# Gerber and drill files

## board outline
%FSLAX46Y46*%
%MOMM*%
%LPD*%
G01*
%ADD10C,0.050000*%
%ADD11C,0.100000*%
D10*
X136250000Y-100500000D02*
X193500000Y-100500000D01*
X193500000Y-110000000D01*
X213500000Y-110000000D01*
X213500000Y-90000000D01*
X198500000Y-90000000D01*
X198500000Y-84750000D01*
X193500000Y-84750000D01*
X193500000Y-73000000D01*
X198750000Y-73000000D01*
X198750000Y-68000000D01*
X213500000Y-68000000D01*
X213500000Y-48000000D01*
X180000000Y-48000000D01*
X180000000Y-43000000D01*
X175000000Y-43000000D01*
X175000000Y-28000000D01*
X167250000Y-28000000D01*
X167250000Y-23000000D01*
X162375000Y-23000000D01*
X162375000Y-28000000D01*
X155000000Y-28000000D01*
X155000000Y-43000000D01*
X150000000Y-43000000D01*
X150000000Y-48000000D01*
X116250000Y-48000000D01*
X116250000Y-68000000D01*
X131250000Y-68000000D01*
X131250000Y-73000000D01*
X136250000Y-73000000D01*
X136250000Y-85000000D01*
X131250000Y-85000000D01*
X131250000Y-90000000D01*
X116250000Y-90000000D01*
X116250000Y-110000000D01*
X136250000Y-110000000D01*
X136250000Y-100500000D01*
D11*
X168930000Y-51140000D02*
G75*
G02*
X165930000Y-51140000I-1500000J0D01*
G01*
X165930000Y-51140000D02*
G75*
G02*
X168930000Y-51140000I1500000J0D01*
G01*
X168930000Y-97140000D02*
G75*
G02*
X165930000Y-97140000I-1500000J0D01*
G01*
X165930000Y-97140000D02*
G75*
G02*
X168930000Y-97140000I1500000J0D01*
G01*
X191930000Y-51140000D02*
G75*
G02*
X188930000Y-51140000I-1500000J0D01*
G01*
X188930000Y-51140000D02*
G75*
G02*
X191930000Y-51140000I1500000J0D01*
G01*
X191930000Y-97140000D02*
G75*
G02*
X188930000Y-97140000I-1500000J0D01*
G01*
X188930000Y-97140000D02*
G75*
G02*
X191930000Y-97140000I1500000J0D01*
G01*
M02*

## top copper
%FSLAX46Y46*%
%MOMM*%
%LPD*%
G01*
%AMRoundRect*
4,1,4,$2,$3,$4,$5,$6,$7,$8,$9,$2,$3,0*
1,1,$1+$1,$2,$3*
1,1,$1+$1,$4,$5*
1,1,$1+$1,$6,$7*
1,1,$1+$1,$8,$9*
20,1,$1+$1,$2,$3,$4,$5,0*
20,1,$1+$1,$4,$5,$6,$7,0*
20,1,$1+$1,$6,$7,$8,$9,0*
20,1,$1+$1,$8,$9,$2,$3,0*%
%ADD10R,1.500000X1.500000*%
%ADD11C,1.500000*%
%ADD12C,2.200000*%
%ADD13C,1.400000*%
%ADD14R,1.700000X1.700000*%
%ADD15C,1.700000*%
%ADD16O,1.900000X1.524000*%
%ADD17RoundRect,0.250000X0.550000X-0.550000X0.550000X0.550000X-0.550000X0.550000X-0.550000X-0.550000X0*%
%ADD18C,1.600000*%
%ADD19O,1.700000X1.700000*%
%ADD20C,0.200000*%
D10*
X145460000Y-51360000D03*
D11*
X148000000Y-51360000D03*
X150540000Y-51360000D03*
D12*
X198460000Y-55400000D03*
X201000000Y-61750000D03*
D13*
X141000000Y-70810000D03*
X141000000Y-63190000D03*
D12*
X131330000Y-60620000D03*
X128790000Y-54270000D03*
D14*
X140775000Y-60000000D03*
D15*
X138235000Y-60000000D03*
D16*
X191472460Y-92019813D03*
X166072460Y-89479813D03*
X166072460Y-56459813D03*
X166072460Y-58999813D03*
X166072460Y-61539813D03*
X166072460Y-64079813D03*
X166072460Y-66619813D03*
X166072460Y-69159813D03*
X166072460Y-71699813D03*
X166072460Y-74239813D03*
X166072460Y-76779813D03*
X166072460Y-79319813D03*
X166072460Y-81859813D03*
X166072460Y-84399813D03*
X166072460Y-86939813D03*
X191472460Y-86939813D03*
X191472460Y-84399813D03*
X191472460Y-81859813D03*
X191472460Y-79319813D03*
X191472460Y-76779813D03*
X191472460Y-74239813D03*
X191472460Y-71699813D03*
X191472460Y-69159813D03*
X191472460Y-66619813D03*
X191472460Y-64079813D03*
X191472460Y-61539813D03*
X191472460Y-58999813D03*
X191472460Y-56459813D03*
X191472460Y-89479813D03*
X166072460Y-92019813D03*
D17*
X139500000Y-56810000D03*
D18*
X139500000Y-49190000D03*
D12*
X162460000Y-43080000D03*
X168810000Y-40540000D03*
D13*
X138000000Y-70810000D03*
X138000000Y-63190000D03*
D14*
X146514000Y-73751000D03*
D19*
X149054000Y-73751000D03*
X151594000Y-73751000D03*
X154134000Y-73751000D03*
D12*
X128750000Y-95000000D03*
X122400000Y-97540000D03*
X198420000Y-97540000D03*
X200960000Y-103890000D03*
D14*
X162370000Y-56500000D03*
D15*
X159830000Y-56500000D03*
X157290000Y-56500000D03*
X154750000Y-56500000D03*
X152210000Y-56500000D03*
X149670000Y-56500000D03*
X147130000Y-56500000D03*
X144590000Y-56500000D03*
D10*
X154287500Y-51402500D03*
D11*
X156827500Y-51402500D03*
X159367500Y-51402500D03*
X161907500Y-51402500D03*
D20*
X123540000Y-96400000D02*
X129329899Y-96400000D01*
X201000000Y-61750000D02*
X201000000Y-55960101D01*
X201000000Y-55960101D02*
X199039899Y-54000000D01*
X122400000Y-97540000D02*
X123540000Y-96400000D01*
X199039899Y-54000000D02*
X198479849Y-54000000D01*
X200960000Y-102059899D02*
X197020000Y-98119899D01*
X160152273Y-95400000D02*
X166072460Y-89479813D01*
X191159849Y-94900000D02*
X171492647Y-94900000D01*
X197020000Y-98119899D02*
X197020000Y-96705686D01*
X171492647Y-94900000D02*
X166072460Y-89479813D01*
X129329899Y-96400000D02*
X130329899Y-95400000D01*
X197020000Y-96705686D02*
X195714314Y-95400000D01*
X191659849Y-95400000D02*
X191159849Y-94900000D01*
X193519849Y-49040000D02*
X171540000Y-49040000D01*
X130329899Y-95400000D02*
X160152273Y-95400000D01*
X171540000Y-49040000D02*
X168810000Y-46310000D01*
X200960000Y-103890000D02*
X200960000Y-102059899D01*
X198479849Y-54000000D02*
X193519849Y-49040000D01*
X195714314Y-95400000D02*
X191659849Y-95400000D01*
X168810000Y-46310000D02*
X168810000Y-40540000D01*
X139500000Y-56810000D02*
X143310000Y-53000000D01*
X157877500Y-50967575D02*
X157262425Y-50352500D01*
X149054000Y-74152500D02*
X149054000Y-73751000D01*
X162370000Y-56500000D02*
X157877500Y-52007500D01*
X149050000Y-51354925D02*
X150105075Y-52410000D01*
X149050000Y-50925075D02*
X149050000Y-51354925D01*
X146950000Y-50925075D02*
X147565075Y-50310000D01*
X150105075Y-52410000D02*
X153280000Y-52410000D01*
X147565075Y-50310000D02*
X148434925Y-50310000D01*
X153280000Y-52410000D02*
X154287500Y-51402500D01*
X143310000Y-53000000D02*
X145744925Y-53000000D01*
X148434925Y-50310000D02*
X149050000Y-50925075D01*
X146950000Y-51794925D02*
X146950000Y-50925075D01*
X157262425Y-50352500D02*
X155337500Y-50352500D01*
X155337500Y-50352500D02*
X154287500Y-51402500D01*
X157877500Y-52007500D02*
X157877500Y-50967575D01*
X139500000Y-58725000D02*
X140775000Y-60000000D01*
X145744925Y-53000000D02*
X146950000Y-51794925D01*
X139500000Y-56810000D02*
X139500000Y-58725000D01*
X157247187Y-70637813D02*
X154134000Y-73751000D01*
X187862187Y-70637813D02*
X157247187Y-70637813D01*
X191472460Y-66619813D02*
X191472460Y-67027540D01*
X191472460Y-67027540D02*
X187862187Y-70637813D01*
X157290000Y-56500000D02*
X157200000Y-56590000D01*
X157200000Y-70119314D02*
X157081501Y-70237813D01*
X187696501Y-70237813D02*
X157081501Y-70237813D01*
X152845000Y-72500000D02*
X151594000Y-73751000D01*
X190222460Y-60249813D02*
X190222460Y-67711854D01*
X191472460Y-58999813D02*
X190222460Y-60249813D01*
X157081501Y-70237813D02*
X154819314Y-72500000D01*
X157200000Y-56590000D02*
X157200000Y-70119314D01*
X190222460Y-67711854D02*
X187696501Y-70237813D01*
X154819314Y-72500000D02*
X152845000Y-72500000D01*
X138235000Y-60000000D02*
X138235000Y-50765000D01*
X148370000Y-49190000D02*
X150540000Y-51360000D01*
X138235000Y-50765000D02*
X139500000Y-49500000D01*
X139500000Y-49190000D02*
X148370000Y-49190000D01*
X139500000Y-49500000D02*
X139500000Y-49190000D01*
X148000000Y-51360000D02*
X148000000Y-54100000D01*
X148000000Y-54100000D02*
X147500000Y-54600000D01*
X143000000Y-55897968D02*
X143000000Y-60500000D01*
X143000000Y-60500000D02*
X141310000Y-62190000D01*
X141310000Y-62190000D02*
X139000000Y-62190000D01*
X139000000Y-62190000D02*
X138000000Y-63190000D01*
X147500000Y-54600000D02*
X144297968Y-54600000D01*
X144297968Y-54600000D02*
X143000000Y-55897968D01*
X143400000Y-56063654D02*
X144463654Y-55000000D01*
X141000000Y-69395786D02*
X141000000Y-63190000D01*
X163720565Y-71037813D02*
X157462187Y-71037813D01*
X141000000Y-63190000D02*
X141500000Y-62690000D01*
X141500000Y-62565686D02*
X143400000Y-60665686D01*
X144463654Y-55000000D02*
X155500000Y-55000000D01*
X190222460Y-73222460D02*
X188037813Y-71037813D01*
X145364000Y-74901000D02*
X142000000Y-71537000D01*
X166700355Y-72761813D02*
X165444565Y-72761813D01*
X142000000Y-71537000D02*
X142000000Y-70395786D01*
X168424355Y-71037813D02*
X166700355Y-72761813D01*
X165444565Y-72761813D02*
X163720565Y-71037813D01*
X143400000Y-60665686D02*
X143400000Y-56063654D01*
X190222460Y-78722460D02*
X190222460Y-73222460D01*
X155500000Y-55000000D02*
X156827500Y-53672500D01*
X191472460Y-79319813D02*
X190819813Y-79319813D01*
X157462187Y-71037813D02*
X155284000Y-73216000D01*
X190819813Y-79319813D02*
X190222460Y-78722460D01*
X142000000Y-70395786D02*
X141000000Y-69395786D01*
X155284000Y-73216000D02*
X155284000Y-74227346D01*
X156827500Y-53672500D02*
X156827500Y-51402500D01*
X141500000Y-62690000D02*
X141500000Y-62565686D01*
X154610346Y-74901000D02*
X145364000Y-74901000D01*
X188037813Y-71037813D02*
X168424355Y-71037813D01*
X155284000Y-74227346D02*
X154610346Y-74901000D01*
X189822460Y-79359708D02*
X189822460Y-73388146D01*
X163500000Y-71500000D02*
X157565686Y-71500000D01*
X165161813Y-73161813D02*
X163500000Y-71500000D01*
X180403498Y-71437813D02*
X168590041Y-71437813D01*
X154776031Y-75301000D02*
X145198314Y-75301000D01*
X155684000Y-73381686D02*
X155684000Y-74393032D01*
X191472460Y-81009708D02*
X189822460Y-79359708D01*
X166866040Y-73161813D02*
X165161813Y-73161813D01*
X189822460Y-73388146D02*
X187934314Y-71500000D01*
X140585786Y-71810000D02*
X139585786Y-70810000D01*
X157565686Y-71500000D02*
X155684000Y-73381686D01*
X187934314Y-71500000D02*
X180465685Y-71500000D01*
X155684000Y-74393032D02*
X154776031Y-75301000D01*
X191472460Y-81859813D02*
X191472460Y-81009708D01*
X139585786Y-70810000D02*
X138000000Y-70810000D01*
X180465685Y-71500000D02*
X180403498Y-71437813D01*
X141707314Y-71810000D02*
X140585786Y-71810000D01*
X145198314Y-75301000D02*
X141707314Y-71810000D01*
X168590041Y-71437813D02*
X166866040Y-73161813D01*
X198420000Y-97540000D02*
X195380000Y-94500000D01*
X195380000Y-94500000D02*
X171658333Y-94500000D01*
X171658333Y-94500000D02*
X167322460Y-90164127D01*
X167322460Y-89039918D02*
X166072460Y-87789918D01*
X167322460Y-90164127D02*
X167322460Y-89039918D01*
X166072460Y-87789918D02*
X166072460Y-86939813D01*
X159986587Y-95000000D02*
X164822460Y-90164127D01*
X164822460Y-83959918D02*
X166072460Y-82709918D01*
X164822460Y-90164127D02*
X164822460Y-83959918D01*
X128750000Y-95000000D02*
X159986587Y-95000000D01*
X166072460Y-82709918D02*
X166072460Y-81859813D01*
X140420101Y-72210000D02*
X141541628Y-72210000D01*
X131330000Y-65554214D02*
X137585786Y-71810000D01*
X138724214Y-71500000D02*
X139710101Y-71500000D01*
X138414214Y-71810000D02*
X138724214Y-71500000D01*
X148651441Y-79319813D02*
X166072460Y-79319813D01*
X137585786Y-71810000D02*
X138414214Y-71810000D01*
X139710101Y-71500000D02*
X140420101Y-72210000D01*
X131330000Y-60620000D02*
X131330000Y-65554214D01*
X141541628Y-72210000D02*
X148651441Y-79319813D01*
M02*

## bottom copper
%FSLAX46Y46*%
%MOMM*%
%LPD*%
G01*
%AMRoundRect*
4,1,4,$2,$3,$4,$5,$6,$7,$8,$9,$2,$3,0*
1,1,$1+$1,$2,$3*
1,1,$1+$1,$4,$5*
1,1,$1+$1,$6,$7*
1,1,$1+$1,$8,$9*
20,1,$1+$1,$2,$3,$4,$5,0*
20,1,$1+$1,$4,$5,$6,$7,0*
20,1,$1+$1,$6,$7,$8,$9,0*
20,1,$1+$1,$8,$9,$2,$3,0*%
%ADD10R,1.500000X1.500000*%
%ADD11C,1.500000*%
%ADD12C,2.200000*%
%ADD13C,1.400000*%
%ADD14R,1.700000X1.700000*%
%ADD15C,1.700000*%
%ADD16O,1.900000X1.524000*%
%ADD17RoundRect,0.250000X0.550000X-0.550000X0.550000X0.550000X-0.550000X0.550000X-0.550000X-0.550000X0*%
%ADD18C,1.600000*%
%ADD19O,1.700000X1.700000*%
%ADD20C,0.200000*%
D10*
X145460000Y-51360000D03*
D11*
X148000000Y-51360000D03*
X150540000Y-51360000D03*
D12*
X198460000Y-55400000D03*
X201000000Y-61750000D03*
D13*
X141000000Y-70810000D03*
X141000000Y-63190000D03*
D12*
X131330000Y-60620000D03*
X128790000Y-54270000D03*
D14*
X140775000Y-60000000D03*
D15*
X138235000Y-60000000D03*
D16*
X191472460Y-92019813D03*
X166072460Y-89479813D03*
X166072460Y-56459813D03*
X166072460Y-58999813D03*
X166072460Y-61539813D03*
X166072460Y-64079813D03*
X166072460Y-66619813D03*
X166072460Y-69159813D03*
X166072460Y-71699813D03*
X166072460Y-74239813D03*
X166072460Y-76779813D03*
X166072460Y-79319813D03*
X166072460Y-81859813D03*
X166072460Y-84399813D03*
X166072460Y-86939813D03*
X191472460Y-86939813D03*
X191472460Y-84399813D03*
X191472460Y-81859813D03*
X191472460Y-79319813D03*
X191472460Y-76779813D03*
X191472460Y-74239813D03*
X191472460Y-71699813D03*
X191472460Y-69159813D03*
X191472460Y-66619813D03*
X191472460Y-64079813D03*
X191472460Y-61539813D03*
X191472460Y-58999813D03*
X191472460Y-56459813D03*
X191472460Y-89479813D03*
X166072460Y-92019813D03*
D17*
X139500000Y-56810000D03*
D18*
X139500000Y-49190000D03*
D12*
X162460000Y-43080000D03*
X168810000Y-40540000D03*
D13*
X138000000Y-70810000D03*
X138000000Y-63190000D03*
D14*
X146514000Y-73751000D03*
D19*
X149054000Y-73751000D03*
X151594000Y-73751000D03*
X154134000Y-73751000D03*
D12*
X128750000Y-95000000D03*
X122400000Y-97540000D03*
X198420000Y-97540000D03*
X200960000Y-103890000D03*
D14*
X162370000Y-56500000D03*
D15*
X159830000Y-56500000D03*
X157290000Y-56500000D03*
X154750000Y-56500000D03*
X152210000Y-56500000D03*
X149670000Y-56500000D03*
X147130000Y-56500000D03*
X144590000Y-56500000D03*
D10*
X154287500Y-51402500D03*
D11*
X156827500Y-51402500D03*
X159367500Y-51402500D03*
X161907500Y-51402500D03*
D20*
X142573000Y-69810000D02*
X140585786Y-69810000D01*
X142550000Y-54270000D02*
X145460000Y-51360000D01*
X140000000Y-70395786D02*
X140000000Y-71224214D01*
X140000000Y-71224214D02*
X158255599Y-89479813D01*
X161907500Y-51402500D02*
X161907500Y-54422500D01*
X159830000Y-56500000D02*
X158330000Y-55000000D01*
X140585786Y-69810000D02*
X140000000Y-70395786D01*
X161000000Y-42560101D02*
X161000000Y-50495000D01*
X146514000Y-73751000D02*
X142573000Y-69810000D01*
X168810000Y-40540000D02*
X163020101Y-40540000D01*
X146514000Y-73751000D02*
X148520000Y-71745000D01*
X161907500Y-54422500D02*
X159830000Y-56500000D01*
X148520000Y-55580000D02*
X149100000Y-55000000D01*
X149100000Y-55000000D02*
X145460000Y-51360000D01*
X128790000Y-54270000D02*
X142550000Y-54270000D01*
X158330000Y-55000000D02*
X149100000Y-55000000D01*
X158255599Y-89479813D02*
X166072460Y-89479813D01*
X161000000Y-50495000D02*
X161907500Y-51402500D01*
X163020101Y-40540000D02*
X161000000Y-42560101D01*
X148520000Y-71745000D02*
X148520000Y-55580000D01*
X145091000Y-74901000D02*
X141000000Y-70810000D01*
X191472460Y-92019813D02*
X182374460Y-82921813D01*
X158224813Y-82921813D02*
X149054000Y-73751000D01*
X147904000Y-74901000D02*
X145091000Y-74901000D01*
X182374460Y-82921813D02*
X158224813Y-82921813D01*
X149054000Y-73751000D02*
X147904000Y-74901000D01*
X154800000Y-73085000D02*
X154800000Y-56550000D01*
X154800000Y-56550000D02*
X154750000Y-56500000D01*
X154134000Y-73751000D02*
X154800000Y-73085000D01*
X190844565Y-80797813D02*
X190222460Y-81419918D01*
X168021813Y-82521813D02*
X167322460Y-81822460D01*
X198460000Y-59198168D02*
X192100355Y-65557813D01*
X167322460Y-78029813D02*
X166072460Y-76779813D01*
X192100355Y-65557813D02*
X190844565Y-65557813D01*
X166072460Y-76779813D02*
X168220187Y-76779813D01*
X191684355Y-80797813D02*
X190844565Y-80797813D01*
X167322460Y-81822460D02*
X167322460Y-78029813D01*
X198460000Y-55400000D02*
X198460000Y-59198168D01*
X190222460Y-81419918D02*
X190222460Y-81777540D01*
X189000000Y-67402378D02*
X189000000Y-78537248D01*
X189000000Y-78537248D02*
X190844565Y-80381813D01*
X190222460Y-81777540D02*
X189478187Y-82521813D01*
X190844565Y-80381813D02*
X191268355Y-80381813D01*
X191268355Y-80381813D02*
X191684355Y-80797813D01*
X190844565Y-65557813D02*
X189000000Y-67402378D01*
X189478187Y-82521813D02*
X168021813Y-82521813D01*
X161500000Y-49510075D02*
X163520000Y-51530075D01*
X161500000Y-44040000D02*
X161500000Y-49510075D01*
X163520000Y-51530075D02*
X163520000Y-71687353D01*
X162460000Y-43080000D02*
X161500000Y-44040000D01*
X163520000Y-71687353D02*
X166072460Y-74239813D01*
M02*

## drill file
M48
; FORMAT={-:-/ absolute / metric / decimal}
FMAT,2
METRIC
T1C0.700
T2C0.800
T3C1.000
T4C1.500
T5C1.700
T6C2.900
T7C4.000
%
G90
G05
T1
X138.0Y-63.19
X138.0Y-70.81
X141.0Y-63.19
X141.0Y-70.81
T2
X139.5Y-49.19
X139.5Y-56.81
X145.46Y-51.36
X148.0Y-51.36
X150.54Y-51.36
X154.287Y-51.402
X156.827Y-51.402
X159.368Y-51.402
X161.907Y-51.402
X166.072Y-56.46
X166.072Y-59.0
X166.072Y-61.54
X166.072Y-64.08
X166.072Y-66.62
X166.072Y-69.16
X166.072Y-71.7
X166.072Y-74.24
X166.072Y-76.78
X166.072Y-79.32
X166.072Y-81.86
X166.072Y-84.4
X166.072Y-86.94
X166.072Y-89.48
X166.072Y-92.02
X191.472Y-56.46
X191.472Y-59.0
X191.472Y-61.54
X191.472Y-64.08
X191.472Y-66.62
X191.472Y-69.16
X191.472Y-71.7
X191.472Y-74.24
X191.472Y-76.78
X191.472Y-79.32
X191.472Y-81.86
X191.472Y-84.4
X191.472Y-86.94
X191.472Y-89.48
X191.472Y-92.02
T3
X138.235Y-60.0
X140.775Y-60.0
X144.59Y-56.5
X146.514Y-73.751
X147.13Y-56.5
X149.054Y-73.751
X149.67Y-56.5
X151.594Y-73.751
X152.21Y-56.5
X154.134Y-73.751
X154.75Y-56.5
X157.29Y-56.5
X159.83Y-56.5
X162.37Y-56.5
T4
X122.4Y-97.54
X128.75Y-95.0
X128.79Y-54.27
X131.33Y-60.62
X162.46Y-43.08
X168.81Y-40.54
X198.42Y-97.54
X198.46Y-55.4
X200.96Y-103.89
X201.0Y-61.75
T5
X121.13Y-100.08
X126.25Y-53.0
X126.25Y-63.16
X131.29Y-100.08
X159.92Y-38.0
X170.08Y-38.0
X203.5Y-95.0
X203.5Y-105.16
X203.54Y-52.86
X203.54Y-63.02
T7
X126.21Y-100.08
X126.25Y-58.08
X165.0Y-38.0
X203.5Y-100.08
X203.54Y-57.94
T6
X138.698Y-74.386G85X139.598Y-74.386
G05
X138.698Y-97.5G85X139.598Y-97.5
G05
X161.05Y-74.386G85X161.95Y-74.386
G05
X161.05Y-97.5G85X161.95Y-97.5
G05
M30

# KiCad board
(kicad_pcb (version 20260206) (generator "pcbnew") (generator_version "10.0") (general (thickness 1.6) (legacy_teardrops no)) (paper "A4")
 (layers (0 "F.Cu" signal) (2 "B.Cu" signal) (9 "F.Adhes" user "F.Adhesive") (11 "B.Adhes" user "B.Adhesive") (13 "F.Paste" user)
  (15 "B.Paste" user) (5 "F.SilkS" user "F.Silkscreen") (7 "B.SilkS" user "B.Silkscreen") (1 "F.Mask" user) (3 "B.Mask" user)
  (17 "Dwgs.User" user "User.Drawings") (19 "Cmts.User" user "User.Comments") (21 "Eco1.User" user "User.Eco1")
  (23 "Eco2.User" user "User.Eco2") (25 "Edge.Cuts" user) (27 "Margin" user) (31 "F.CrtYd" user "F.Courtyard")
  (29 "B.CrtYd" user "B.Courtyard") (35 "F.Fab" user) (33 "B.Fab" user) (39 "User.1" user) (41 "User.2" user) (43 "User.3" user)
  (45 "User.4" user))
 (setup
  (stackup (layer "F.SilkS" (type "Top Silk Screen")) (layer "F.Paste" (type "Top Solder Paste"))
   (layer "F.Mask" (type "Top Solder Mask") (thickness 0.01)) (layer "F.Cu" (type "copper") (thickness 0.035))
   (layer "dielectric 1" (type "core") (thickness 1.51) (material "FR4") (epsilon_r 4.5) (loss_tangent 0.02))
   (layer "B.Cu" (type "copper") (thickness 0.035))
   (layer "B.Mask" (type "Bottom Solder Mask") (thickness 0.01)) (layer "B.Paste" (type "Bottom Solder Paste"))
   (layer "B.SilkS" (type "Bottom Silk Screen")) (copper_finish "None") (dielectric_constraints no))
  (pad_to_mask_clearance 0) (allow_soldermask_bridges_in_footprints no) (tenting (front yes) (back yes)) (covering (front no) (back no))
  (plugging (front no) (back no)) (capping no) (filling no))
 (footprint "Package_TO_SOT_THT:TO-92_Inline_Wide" (layer "F.Cu") (at 145.46 51.36)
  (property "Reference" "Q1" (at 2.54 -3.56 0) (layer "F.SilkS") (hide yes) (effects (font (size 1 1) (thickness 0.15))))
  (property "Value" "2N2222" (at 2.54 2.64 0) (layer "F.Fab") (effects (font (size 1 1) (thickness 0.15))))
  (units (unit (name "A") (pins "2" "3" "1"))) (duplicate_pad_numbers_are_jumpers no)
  (pad "1" thru_hole rect (at 0 0) (size 1.5 1.5) (drill 0.8) (layers "*.Cu" "*.Mask") (remove_unused_layers no) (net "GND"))
  (pad "2" thru_hole circle (at 2.54 0) (size 1.5 1.5) (drill 0.8) (layers "*.Cu" "*.Mask") (remove_unused_layers no) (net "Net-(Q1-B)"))
  (pad "3" thru_hole circle (at 5.08 0) (size 1.5 1.5) (drill 0.8) (layers "*.Cu" "*.Mask") (remove_unused_layers no) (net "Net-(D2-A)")))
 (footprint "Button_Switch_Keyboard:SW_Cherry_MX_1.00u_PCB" (layer "F.Cu") (at 198.46 55.4 90)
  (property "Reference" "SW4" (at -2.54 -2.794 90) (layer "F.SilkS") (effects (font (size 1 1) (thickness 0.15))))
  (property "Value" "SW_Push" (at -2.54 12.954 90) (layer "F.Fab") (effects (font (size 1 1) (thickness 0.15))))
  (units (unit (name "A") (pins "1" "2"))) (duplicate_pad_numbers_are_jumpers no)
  (pad "" np_thru_hole circle (at -7.62 5.08 90) (size 1.7 1.7) (drill 1.7) (layers "*.Cu" "*.Mask"))
  (pad "" np_thru_hole circle (at -2.54 5.08 90) (size 4 4) (drill 4) (layers "*.Cu" "*.Mask"))
  (pad "" np_thru_hole circle (at 2.54 5.08 90) (size 1.7 1.7) (drill 1.7) (layers "*.Cu" "*.Mask"))
  (pad "1" thru_hole circle (at 0 0 90) (size 2.2 2.2) (drill 1.5) (layers "*.Cu" "*.Mask") (remove_unused_layers no) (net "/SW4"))
  (pad "2" thru_hole circle (at -6.35 2.54 90) (size 2.2 2.2) (drill 1.5) (layers "*.Cu" "*.Mask") (remove_unused_layers no) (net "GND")))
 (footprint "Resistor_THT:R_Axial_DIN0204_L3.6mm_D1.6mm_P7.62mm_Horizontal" (layer "F.Cu") (at 141 70.81 90)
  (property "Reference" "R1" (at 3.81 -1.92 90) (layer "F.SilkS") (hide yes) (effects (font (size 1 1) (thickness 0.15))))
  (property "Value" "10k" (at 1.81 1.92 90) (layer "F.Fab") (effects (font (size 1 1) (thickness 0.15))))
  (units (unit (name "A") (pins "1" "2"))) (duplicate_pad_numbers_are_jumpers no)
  (pad "1" thru_hole circle (at 0 0 90) (size 1.4 1.4) (drill 0.7) (layers "*.Cu" "*.Mask") (remove_unused_layers no) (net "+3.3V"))
  (pad "2" thru_hole circle (at 7.62 0 90) (size 1.4 1.4) (drill 0.7) (layers "*.Cu" "*.Mask") (remove_unused_layers no) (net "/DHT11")))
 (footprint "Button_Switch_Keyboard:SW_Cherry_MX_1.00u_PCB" (layer "F.Cu") (at 131.33 60.62 -90)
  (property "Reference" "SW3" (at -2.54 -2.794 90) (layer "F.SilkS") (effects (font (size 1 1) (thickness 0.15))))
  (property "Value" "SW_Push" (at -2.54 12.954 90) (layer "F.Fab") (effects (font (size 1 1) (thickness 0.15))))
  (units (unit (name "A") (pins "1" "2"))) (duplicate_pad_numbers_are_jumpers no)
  (pad "" np_thru_hole circle (at -7.62 5.08 270) (size 1.7 1.7) (drill 1.7) (layers "*.Cu" "*.Mask"))
  (pad "" np_thru_hole circle (at -2.54 5.08 270) (size 4 4) (drill 4) (layers "*.Cu" "*.Mask"))
  (pad "" np_thru_hole circle (at 2.54 5.08 270) (size 1.7 1.7) (drill 1.7) (layers "*.Cu" "*.Mask"))
  (pad "1" thru_hole circle (at 0 0 270) (size 2.2 2.2) (drill 1.5) (layers "*.Cu" "*.Mask") (remove_unused_layers no) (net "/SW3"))
  (pad "2" thru_hole circle (at -6.35 2.54 270) (size 2.2 2.2) (drill 1.5) (layers "*.Cu" "*.Mask") (remove_unused_layers no) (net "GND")))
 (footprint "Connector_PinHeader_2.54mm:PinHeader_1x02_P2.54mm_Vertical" (layer "F.Cu") (at 140.775 60 -90)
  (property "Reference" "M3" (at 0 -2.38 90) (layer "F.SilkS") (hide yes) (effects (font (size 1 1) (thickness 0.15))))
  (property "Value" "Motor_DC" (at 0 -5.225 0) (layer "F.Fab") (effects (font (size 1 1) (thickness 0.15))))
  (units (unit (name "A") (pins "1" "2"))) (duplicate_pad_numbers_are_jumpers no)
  (pad "1" thru_hole rect (at 0 0 270) (size 1.7 1.7) (drill 1) (layers "*.Cu" "*.Mask") (remove_unused_layers no) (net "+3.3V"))
  (pad "2" thru_hole circle (at 0 2.54 270) (size 1.7 1.7) (drill 1) (layers "*.Cu" "*.Mask") (remove_unused_layers no) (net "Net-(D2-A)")))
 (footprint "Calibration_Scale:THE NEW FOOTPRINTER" (layer "F.Cu") (at 178 75)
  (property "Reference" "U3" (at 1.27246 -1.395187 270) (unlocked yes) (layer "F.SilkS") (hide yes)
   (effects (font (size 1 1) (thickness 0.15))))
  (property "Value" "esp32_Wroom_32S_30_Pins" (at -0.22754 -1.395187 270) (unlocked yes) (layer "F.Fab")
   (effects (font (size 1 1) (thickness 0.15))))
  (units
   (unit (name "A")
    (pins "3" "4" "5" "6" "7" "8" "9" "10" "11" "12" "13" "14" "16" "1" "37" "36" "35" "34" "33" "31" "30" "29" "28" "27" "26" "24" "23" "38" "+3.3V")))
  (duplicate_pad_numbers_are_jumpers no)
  (fp_circle (center -10.57 -23.86) (end -10.57 -22.36) (stroke (width 0.1) (type default)) (fill no) (layer "Edge.Cuts"))
  (fp_circle (center -10.57 22.14) (end -10.57 23.64) (stroke (width 0.1) (type default)) (fill no) (layer "Edge.Cuts"))
  (fp_circle (center 12.43 -23.86) (end 12.43 -22.36) (stroke (width 0.1) (type default)) (fill no) (layer "Edge.Cuts"))
  (fp_circle (center 12.43 22.14) (end 12.43 23.64) (stroke (width 0.1) (type default)) (fill no) (layer "Edge.Cuts"))
  (pad "+3.3V" thru_hole oval (at 13.47246 17.019813 270) (size 1.524 1.9) (drill 0.8) (layers "*.Cu" "*.Mask") (remove_unused_layers no)
   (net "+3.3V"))
  (pad "1" thru_hole oval (at -11.92754 14.479813 270) (size 1.524 1.9) (drill 0.8) (layers "*.Cu" "*.Mask") (remove_unused_layers no)
   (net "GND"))
  (pad "3" thru_hole oval (at -11.92754 -18.540187 270) (size 1.524 1.9) (drill 0.8) (layers "*.Cu" "*.Mask") (remove_unused_layers no)
   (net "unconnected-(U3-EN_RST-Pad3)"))
  (pad "4" thru_hole oval (at -11.92754 -16.000187 270) (size 1.524 1.9) (drill 0.8) (layers "*.Cu" "*.Mask") (remove_unused_layers no)
   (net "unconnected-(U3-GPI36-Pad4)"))
  (pad "5" thru_hole oval (at -11.92754 -13.460187 270) (size 1.524 1.9) (drill 0.8) (layers "*.Cu" "*.Mask") (remove_unused_layers no)
   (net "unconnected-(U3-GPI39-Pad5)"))
  (pad "6" thru_hole oval (at -11.92754 -10.920187 270) (size 1.524 1.9) (drill 0.8) (layers "*.Cu" "*.Mask") (remove_unused_layers no)
   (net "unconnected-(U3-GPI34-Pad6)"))
  (pad "7" thru_hole oval (at -11.92754 -8.380187 270) (size 1.524 1.9) (drill 0.8) (layers "*.Cu" "*.Mask") (remove_unused_layers no)
   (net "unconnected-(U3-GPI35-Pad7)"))
  (pad "8" thru_hole oval (at -11.92754 -5.840187 270) (size 1.524 1.9) (drill 0.8) (layers "*.Cu" "*.Mask") (remove_unused_layers no)
   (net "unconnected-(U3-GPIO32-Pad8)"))
  (pad "9" thru_hole oval (at -11.92754 -3.300187 270) (size 1.524 1.9) (drill 0.8) (layers "*.Cu" "*.Mask") (remove_unused_layers no)
   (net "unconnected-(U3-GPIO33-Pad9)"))
  (pad "10" thru_hole oval (at -11.92754 -0.760187 270) (size 1.524 1.9) (drill 0.8) (layers "*.Cu" "*.Mask") (remove_unused_layers no)
   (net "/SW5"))
  (pad "11" thru_hole oval (at -11.92754 1.779813 270) (size 1.524 1.9) (drill 0.8) (layers "*.Cu" "*.Mask") (remove_unused_layers no)
   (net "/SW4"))
  (pad "12" thru_hole oval (at -11.92754 4.319813 270) (size 1.524 1.9) (drill 0.8) (layers "*.Cu" "*.Mask") (remove_unused_layers no)
   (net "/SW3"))
  (pad "13" thru_hole oval (at -11.92754 6.859813 270) (size 1.524 1.9) (drill 0.8) (layers "*.Cu" "*.Mask") (remove_unused_layers no)
   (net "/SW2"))
  (pad "14" thru_hole oval (at -11.92754 9.399813 270) (size 1.524 1.9) (drill 0.8) (layers "*.Cu" "*.Mask") (remove_unused_layers no)
   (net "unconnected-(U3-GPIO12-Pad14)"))
  (pad "16" thru_hole oval (at -11.92754 11.939813 270) (size 1.524 1.9) (drill 0.8) (layers "*.Cu" "*.Mask") (remove_unused_layers no)
   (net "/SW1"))
  (pad "23" thru_hole oval (at 13.47246 11.939813 270) (size 1.524 1.9) (drill 0.8) (layers "*.Cu" "*.Mask") (remove_unused_layers no)
   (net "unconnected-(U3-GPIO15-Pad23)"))
  (pad "24" thru_hole oval (at 13.47246 9.399813 270) (size 1.524 1.9) (drill 0.8) (layers "*.Cu" "*.Mask") (remove_unused_layers no)
   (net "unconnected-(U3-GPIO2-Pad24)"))
  (pad "26" thru_hole oval (at 13.47246 6.859813 270) (size 1.524 1.9) (drill 0.8) (layers "*.Cu" "*.Mask" "Dwgs.User")
   (remove_unused_layers no) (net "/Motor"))
  (pad "27" thru_hole oval (at 13.47246 4.319813 270) (size 1.524 1.9) (drill 0.8) (layers "*.Cu" "*.Mask") (remove_unused_layers no)
   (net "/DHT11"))
  (pad "28" thru_hole oval (at 13.47246 1.779813 270) (size 1.524 1.9) (drill 0.8) (layers "*.Cu" "*.Mask") (remove_unused_layers no)
   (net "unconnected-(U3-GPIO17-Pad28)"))
  (pad "29" thru_hole oval (at 13.47246 -0.760187 270) (size 1.524 1.9) (drill 0.8) (layers "*.Cu" "*.Mask") (remove_unused_layers no)
   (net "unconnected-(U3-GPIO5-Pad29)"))
  (pad "30" thru_hole oval (at 13.47246 -3.300187 270) (size 1.524 1.9) (drill 0.8) (layers "*.Cu" "*.Mask") (remove_unused_layers no)
   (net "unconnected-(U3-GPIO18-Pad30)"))
  (pad "31" thru_hole oval (at 13.47246 -5.840187 270) (size 1.524 1.9) (drill 0.8) (layers "*.Cu" "*.Mask") (remove_unused_layers no)
   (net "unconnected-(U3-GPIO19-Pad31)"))
  (pad "33" thru_hole oval (at 13.47246 -8.380187 270) (size 1.524 1.9) (drill 0.8) (layers "*.Cu" "*.Mask") (remove_unused_layers no)
   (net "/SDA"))
  (pad "34" thru_hole oval (at 13.47246 -10.920187 270) (size 1.524 1.9) (drill 0.8) (layers "*.Cu" "*.Mask") (remove_unused_layers no)
   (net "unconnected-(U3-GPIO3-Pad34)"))
  (pad "35" thru_hole oval (at 13.47246 -13.460187 270) (size 1.524 1.9) (drill 0.8) (layers "*.Cu" "*.Mask") (remove_unused_layers no)
   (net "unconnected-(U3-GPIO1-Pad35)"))
  (pad "36" thru_hole oval (at 13.47246 -16.000187 270) (size 1.524 1.9) (drill 0.8) (layers "*.Cu" "*.Mask") (remove_unused_layers no)
   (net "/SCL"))
  (pad "37" thru_hole oval (at 13.47246 -18.540187 270) (size 1.524 1.9) (drill 0.8) (layers "*.Cu" "*.Mask") (remove_unused_layers no)
   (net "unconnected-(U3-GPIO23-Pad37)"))
  (pad "38" thru_hole oval (at 13.47246 14.479813 270) (size 1.524 1.9) (drill 0.8) (layers "*.Cu" "*.Mask") (remove_unused_layers no)
   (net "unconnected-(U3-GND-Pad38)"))
  (pad "vin" thru_hole oval (at -11.92754 17.019813 270) (size 1.524 1.9) (drill 0.8) (layers "*.Cu" "*.Mask") (remove_unused_layers no)))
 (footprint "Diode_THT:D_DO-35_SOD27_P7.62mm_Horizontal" (layer "F.Cu") (at 139.5 56.81 90)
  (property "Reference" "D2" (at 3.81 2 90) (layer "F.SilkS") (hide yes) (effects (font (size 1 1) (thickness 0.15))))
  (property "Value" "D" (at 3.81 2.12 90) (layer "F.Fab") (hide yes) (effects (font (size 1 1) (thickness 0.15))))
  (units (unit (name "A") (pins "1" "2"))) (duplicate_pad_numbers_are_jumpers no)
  (pad "1" thru_hole roundrect (at 0 0 90) (size 1.6 1.6) (drill 0.8) (layers "*.Cu" "*.Mask") (remove_unused_layers no)
   (roundrect_rratio 0.15625) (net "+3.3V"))
  (pad "2" thru_hole circle (at 7.62 0 90) (size 1.6 1.6) (drill 0.8) (layers "*.Cu" "*.Mask") (remove_unused_layers no) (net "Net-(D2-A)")))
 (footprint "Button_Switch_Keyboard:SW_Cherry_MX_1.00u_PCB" (layer "F.Cu") (at 162.46 43.08 180)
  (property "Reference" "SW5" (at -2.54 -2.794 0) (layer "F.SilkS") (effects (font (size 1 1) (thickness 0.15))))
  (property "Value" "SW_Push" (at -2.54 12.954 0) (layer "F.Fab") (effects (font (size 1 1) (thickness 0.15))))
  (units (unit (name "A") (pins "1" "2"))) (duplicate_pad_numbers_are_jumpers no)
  (pad "" np_thru_hole circle (at -7.62 5.08 180) (size 1.7 1.7) (drill 1.7) (layers "*.Cu" "*.Mask"))
  (pad "" np_thru_hole circle (at -2.54 5.08 180) (size 4 4) (drill 4) (layers "*.Cu" "*.Mask"))
  (pad "" np_thru_hole circle (at 2.54 5.08 180) (size 1.7 1.7) (drill 1.7) (layers "*.Cu" "*.Mask"))
  (pad "1" thru_hole circle (at 0 0 180) (size 2.2 2.2) (drill 1.5) (layers "*.Cu" "*.Mask") (remove_unused_layers no) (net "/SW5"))
  (pad "2" thru_hole circle (at -6.35 2.54 180) (size 2.2 2.2) (drill 1.5) (layers "*.Cu" "*.Mask") (remove_unused_layers no) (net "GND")))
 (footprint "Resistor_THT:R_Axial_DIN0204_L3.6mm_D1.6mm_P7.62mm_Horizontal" (layer "F.Cu") (at 138 70.81 90)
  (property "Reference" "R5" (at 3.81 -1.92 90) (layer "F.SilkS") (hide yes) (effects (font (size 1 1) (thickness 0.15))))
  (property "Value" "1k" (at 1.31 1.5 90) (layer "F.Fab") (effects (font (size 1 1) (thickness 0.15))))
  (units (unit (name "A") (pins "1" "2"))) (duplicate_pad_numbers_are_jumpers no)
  (pad "1" thru_hole circle (at 0 0 90) (size 1.4 1.4) (drill 0.7) (layers "*.Cu" "*.Mask") (remove_unused_layers no) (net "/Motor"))
  (pad "2" thru_hole circle (at 7.62 0 90) (size 1.4 1.4) (drill 0.7) (layers "*.Cu" "*.Mask") (remove_unused_layers no) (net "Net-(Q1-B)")))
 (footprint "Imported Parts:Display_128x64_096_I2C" (layer "F.Cu") (at 150.324 73.751)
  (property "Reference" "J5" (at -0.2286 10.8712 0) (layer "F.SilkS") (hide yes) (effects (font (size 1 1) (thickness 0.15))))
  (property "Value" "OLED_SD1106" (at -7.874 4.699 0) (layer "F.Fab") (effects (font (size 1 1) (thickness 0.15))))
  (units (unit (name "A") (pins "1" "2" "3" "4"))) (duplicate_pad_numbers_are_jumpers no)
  (pad "" np_thru_hole oval (at -11.176 0.635) (size 3.8 2.9) (drill oval 3.8 2.9) (layers "*.Cu" "*.Mask"))
  (pad "" np_thru_hole oval (at -11.176 23.749) (size 3.8 2.9) (drill oval 3.8 2.9) (layers "*.Cu" "*.Mask"))
  (pad "" np_thru_hole oval (at 11.176 0.635) (size 3.8 2.9) (drill oval 3.8 2.9) (layers "*.Cu" "*.Mask"))
  (pad "" np_thru_hole oval (at 11.176 23.749) (size 3.8 2.9) (drill oval 3.8 2.9) (layers "*.Cu" "*.Mask"))
  (pad "1" thru_hole rect (at -3.81 0 90) (size 1.7 1.7) (drill 1) (layers "*.Cu" "*.Mask") (remove_unused_layers no) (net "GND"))
  (pad "2" thru_hole oval (at -1.27 0 90) (size 1.7 1.7) (drill 1) (layers "*.Cu" "*.Mask") (remove_unused_layers no) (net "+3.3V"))
  (pad "3" thru_hole oval (at 1.27 0 90) (size 1.7 1.7) (drill 1) (layers "*.Cu" "*.Mask") (remove_unused_layers no) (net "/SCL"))
  (pad "4" thru_hole oval (at 3.81 0 90) (size 1.7 1.7) (drill 1) (layers "*.Cu" "*.Mask") (remove_unused_layers no) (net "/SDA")))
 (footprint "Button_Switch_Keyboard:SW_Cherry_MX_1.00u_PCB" (layer "F.Cu") (at 128.75 95)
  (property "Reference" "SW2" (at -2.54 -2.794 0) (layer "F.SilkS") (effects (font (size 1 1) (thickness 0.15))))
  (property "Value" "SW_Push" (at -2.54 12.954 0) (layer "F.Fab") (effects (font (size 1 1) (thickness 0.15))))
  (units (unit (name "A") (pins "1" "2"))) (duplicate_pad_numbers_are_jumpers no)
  (pad "" np_thru_hole circle (at -7.62 5.08) (size 1.7 1.7) (drill 1.7) (layers "*.Cu" "*.Mask"))
  (pad "" np_thru_hole circle (at -2.54 5.08) (size 4 4) (drill 4) (layers "*.Cu" "*.Mask"))
  (pad "" np_thru_hole circle (at 2.54 5.08) (size 1.7 1.7) (drill 1.7) (layers "*.Cu" "*.Mask"))
  (pad "1" thru_hole circle (at 0 0) (size 2.2 2.2) (drill 1.5) (layers "*.Cu" "*.Mask") (remove_unused_layers no) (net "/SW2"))
  (pad "2" thru_hole circle (at -6.35 2.54) (size 2.2 2.2) (drill 1.5) (layers "*.Cu" "*.Mask") (remove_unused_layers no) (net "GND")))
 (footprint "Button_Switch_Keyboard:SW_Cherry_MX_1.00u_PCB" (layer "F.Cu") (at 198.42 97.54 90)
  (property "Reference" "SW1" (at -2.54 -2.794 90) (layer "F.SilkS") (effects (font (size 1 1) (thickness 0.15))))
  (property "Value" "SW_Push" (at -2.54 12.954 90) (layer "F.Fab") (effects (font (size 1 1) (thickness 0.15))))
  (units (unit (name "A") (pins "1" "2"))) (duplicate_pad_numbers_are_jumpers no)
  (pad "" np_thru_hole circle (at -7.62 5.08 90) (size 1.7 1.7) (drill 1.7) (layers "*.Cu" "*.Mask"))
  (pad "" np_thru_hole circle (at -2.54 5.08 90) (size 4 4) (drill 4) (layers "*.Cu" "*.Mask"))
  (pad "" np_thru_hole circle (at 2.54 5.08 90) (size 1.7 1.7) (drill 1.7) (layers "*.Cu" "*.Mask"))
  (pad "1" thru_hole circle (at 0 0 90) (size 2.2 2.2) (drill 1.5) (layers "*.Cu" "*.Mask") (remove_unused_layers no) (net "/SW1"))
  (pad "2" thru_hole circle (at -6.35 2.54 90) (size 2.2 2.2) (drill 1.5) (layers "*.Cu" "*.Mask") (remove_unused_layers no) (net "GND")))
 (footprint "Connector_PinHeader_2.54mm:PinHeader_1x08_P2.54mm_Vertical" (layer "F.Cu") (at 162.37 56.5 -90)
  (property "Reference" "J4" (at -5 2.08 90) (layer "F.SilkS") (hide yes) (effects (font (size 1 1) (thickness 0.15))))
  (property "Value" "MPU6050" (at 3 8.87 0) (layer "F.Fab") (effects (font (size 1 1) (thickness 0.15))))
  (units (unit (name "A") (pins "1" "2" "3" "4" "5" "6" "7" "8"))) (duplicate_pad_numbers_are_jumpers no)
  (pad "1" thru_hole rect (at 0 0 270) (size 1.7 1.7) (drill 1) (layers "*.Cu" "*.Mask") (remove_unused_layers no) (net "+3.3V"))
  (pad "2" thru_hole circle (at 0 2.54 270) (size 1.7 1.7) (drill 1) (layers "*.Cu" "*.Mask") (remove_unused_layers no) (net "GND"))
  (pad "3" thru_hole circle (at 0 5.08 270) (size 1.7 1.7) (drill 1) (layers "*.Cu" "*.Mask") (remove_unused_layers no) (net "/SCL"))
  (pad "4" thru_hole circle (at 0 7.62 270) (size 1.7 1.7) (drill 1) (layers "*.Cu" "*.Mask") (remove_unused_layers no) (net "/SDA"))
  (pad "5" thru_hole circle (at 0 10.16 270) (size 1.7 1.7) (drill 1) (layers "*.Cu" "*.Mask") (remove_unused_layers no)
   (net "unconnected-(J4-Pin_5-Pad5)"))
  (pad "6" thru_hole circle (at 0 12.7 270) (size 1.7 1.7) (drill 1) (layers "*.Cu" "*.Mask") (remove_unused_layers no)
   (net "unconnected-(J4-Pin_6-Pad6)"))
  (pad "7" thru_hole circle (at 0 15.24 270) (size 1.7 1.7) (drill 1) (layers "*.Cu" "*.Mask") (remove_unused_layers no)
   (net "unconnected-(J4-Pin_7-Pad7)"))
  (pad "8" thru_hole circle (at 0 17.78 270) (size 1.7 1.7) (drill 1) (layers "*.Cu" "*.Mask") (remove_unused_layers no)
   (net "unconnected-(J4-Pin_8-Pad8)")))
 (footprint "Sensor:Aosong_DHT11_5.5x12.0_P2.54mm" (layer "F.Cu") (at 154.2875 51.4025 90)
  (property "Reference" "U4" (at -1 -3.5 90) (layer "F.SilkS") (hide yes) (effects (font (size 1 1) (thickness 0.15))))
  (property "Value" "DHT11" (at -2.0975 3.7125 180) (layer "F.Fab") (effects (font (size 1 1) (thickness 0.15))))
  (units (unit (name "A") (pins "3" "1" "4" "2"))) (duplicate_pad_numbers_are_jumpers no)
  (pad "1" thru_hole rect (at 0 0 90) (size 1.5 1.5) (drill 0.8) (layers "*.Cu" "*.Mask") (remove_unused_layers no) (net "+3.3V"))
  (pad "2" thru_hole circle (at 0 2.54 90) (size 1.5 1.5) (drill 0.8) (layers "*.Cu" "*.Mask") (remove_unused_layers no) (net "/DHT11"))
  (pad "3" thru_hole circle (at 0 5.08 90) (size 1.5 1.5) (drill 0.8) (layers "*.Cu" "*.Mask") (remove_unused_layers no)
   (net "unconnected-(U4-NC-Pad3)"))
  (pad "4" thru_hole circle (at 0 7.62 90) (size 1.5 1.5) (drill 0.8) (layers "*.Cu" "*.Mask") (remove_unused_layers no) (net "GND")))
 (gr_poly
  (pts (xy 136.25 100.5) (xy 193.5 100.5) (xy 193.5 110) (xy 213.5 110) (xy 213.5 90) (xy 198.5 90) (xy 198.5 84.75) (xy 193.5 84.75)
   (xy 193.5 73) (xy 198.75 73) (xy 198.75 68) (xy 213.5 68) (xy 213.5 48) (xy 180 48) (xy 180 43) (xy 175 43) (xy 175 28) (xy 167.25 28)
   (xy 167.25 23) (xy 162.375 23) (xy 162.375 28) (xy 155 28) (xy 155 43) (xy 150 43) (xy 150 48) (xy 116.25 48) (xy 116.25 68)
   (xy 131.25 68) (xy 131.25 73) (xy 136.25 73) (xy 136.25 85) (xy 131.25 85) (xy 131.25 90) (xy 116.25 90) (xy 116.25 110) (xy 136.25 110))
  (stroke (width 0.05) (type solid)) (fill no) (layer "Edge.Cuts"))
 (segment (start 123.54 96.4) (end 129.329899 96.4) (width 0.2) (layer "F.Cu") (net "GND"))
 (segment (start 201 61.75) (end 201 55.960101) (width 0.2) (layer "F.Cu") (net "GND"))
 (segment (start 201 55.960101) (end 199.039899 54) (width 0.2) (layer "F.Cu") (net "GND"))
 (segment (start 122.4 97.54) (end 123.54 96.4) (width 0.2) (layer "F.Cu") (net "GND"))
 (segment (start 199.039899 54) (end 198.479849 54) (width 0.2) (layer "F.Cu") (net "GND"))
 (segment (start 200.96 102.059899) (end 197.02 98.119899) (width 0.2) (layer "F.Cu") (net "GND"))
 (segment (start 160.152273 95.4) (end 166.07246 89.479813) (width 0.2) (layer "F.Cu") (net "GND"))
 (segment (start 191.159849 94.9) (end 171.492647 94.9) (width 0.2) (layer "F.Cu") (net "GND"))
 (segment (start 197.02 98.119899) (end 197.02 96.705686) (width 0.2) (layer "F.Cu") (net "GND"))
 (segment (start 171.492647 94.9) (end 166.07246 89.479813) (width 0.2) (layer "F.Cu") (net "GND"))
 (segment (start 129.329899 96.4) (end 130.329899 95.4) (width 0.2) (layer "F.Cu") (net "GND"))
 (segment (start 197.02 96.705686) (end 195.714314 95.4) (width 0.2) (layer "F.Cu") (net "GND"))
 (segment (start 191.659849 95.4) (end 191.159849 94.9) (width 0.2) (layer "F.Cu") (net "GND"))
 (segment (start 193.519849 49.04) (end 171.54 49.04) (width 0.2) (layer "F.Cu") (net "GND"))
 (segment (start 130.329899 95.4) (end 160.152273 95.4) (width 0.2) (layer "F.Cu") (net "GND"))
 (segment (start 171.54 49.04) (end 168.81 46.31) (width 0.2) (layer "F.Cu") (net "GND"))
 (segment (start 200.96 103.89) (end 200.96 102.059899) (width 0.2) (layer "F.Cu") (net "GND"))
 (segment (start 198.479849 54) (end 193.519849 49.04) (width 0.2) (layer "F.Cu") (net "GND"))
 (segment (start 195.714314 95.4) (end 191.659849 95.4) (width 0.2) (layer "F.Cu") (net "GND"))
 (segment (start 168.81 46.31) (end 168.81 40.54) (width 0.2) (layer "F.Cu") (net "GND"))
 (segment (start 142.573 69.81) (end 140.585786 69.81) (width 0.2) (layer "B.Cu") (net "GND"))
 (segment (start 142.55 54.27) (end 145.46 51.36) (width 0.2) (layer "B.Cu") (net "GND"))
 (segment (start 140 70.395786) (end 140 71.224214) (width 0.2) (layer "B.Cu") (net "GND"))
 (segment (start 140 71.224214) (end 158.255599 89.479813) (width 0.2) (layer "B.Cu") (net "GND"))
 (segment (start 161.9075 51.4025) (end 161.9075 54.4225) (width 0.2) (layer "B.Cu") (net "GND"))
 (segment (start 159.83 56.5) (end 158.33 55) (width 0.2) (layer "B.Cu") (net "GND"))
 (segment (start 140.585786 69.81) (end 140 70.395786) (width 0.2) (layer "B.Cu") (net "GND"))
 (segment (start 161 42.560101) (end 161 50.495) (width 0.2) (layer "B.Cu") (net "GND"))
 (segment (start 146.514 73.751) (end 142.573 69.81) (width 0.2) (layer "B.Cu") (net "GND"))
 (segment (start 168.81 40.54) (end 163.020101 40.54) (width 0.2) (layer "B.Cu") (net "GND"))
 (segment (start 146.514 73.751) (end 148.52 71.745) (width 0.2) (layer "B.Cu") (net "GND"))
 (segment (start 161.9075 54.4225) (end 159.83 56.5) (width 0.2) (layer "B.Cu") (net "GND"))
 (segment (start 148.52 55.58) (end 149.1 55) (width 0.2) (layer "B.Cu") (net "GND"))
 (segment (start 149.1 55) (end 145.46 51.36) (width 0.2) (layer "B.Cu") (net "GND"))
 (segment (start 128.79 54.27) (end 142.55 54.27) (width 0.2) (layer "B.Cu") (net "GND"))
 (segment (start 158.33 55) (end 149.1 55) (width 0.2) (layer "B.Cu") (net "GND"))
 (segment (start 158.255599 89.479813) (end 166.07246 89.479813) (width 0.2) (layer "B.Cu") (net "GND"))
 (segment (start 161 50.495) (end 161.9075 51.4025) (width 0.2) (layer "B.Cu") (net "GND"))
 (segment (start 163.020101 40.54) (end 161 42.560101) (width 0.2) (layer "B.Cu") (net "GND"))
 (segment (start 148.52 71.745) (end 148.52 55.58) (width 0.2) (layer "B.Cu") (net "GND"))
 (segment (start 139.5 56.81) (end 143.31 53) (width 0.2) (layer "F.Cu") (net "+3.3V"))
 (segment (start 157.8775 50.967575) (end 157.262425 50.3525) (width 0.2) (layer "F.Cu") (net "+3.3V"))
 (segment (start 149.054 74.1525) (end 149.054 73.751) (width 0.2) (layer "F.Cu") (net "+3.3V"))
 (segment (start 162.37 56.5) (end 157.8775 52.0075) (width 0.2) (layer "F.Cu") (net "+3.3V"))
 (segment (start 149.05 51.354925) (end 150.105075 52.41) (width 0.2) (layer "F.Cu") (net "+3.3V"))
 (segment (start 149.05 50.925075) (end 149.05 51.354925) (width 0.2) (layer "F.Cu") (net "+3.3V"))
 (segment (start 146.95 50.925075) (end 147.565075 50.31) (width 0.2) (layer "F.Cu") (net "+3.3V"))
 (segment (start 150.105075 52.41) (end 153.28 52.41) (width 0.2) (layer "F.Cu") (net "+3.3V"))
 (segment (start 147.565075 50.31) (end 148.434925 50.31) (width 0.2) (layer "F.Cu") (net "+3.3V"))
 (segment (start 153.28 52.41) (end 154.2875 51.4025) (width 0.2) (layer "F.Cu") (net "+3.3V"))
 (segment (start 143.31 53) (end 145.744925 53) (width 0.2) (layer "F.Cu") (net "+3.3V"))
 (segment (start 148.434925 50.31) (end 149.05 50.925075) (width 0.2) (layer "F.Cu") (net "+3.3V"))
 (segment (start 146.95 51.794925) (end 146.95 50.925075) (width 0.2) (layer "F.Cu") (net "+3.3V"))
 (segment (start 157.262425 50.3525) (end 155.3375 50.3525) (width 0.2) (layer "F.Cu") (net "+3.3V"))
 (segment (start 155.3375 50.3525) (end 154.2875 51.4025) (width 0.2) (layer "F.Cu") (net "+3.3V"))
 (segment (start 157.8775 52.0075) (end 157.8775 50.967575) (width 0.2) (layer "F.Cu") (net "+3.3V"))
 (segment (start 139.5 58.725) (end 140.775 60) (width 0.2) (layer "F.Cu") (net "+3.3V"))
 (segment (start 145.744925 53) (end 146.95 51.794925) (width 0.2) (layer "F.Cu") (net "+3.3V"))
 (segment (start 139.5 56.81) (end 139.5 58.725) (width 0.2) (layer "F.Cu") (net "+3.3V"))
 (segment (start 145.091 74.901) (end 141 70.81) (width 0.2) (layer "B.Cu") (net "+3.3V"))
 (segment (start 191.47246 92.019813) (end 182.37446 82.921813) (width 0.2) (layer "B.Cu") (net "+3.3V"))
 (segment (start 158.224813 82.921813) (end 149.054 73.751) (width 0.2) (layer "B.Cu") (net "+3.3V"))
 (segment (start 147.904 74.901) (end 145.091 74.901) (width 0.2) (layer "B.Cu") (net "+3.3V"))
 (segment (start 182.37446 82.921813) (end 158.224813 82.921813) (width 0.2) (layer "B.Cu") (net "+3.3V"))
 (segment (start 149.054 73.751) (end 147.904 74.901) (width 0.2) (layer "B.Cu") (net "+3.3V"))
 (segment (start 157.247187 70.637813) (end 154.134 73.751) (width 0.2) (layer "F.Cu") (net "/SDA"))
 (segment (start 187.862187 70.637813) (end 157.247187 70.637813) (width 0.2) (layer "F.Cu") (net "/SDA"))
 (segment (start 191.47246 66.619813) (end 191.47246 67.02754) (width 0.2) (layer "F.Cu") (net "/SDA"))
 (segment (start 191.47246 67.02754) (end 187.862187 70.637813) (width 0.2) (layer "F.Cu") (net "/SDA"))
 (segment (start 154.8 73.085) (end 154.8 56.55) (width 0.2) (layer "B.Cu") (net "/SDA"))
 (segment (start 154.8 56.55) (end 154.75 56.5) (width 0.2) (layer "B.Cu") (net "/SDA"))
 (segment (start 154.134 73.751) (end 154.8 73.085) (width 0.2) (layer "B.Cu") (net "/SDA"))
 (segment (start 157.29 56.5) (end 157.2 56.59) (width 0.2) (layer "F.Cu") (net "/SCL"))
 (segment (start 157.2 70.119314) (end 157.081501 70.237813) (width 0.2) (layer "F.Cu") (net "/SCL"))
 (segment (start 187.696501 70.237813) (end 157.081501 70.237813) (width 0.2) (layer "F.Cu") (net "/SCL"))
 (segment (start 152.845 72.5) (end 151.594 73.751) (width 0.2) (layer "F.Cu") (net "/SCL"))
 (segment (start 190.22246 60.249813) (end 190.22246 67.711854) (width 0.2) (layer "F.Cu") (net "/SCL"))
 (segment (start 191.47246 58.999813) (end 190.22246 60.249813) (width 0.2) (layer "F.Cu") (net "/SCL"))
 (segment (start 157.081501 70.237813) (end 154.819314 72.5) (width 0.2) (layer "F.Cu") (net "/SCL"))
 (segment (start 157.2 56.59) (end 157.2 70.119314) (width 0.2) (layer "F.Cu") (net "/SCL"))
 (segment (start 190.22246 67.711854) (end 187.696501 70.237813) (width 0.2) (layer "F.Cu") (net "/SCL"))
 (segment (start 154.819314 72.5) (end 152.845 72.5) (width 0.2) (layer "F.Cu") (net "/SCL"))
 (segment (start 138.235 60) (end 138.235 50.765) (width 0.2) (layer "F.Cu") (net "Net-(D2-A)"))
 (segment (start 148.37 49.19) (end 150.54 51.36) (width 0.2) (layer "F.Cu") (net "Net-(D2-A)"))
 (segment (start 138.235 50.765) (end 139.5 49.5) (width 0.2) (layer "F.Cu") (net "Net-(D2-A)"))
 (segment (start 139.5 49.19) (end 148.37 49.19) (width 0.2) (layer "F.Cu") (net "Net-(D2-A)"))
 (segment (start 139.5 49.5) (end 139.5 49.19) (width 0.2) (layer "F.Cu") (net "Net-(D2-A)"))
 (segment (start 148 51.36) (end 148 54.1) (width 0.2) (layer "F.Cu") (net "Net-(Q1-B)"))
 (segment (start 148 54.1) (end 147.5 54.6) (width 0.2) (layer "F.Cu") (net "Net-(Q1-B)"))
 (segment (start 143 55.897968) (end 143 60.5) (width 0.2) (layer "F.Cu") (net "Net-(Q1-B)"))
 (segment (start 143 60.5) (end 141.31 62.19) (width 0.2) (layer "F.Cu") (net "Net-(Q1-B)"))
 (segment (start 141.31 62.19) (end 139 62.19) (width 0.2) (layer "F.Cu") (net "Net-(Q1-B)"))
 (segment (start 139 62.19) (end 138 63.19) (width 0.2) (layer "F.Cu") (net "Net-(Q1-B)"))
 (segment (start 147.5 54.6) (end 144.297968 54.6) (width 0.2) (layer "F.Cu") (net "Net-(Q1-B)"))
 (segment (start 144.297968 54.6) (end 143 55.897968) (width 0.2) (layer "F.Cu") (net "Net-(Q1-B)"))
 (segment (start 143.4 56.063654) (end 144.463654 55) (width 0.2) (layer "F.Cu") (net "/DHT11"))
 (segment (start 141 69.395786) (end 141 63.19) (width 0.2) (layer "F.Cu") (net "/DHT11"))
 (segment (start 163.720565 71.037813) (end 157.462187 71.037813) (width 0.2) (layer "F.Cu") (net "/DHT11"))
 (segment (start 141 63.19) (end 141.5 62.69) (width 0.2) (layer "F.Cu") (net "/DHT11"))
 (segment (start 141.5 62.565686) (end 143.4 60.665686) (width 0.2) (layer "F.Cu") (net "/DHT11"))
 (segment (start 144.463654 55) (end 155.5 55) (width 0.2) (layer "F.Cu") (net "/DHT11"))
 (segment (start 190.22246 73.22246) (end 188.037813 71.037813) (width 0.2) (layer "F.Cu") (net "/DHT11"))
 (segment (start 145.364 74.901) (end 142 71.537) (width 0.2) (layer "F.Cu") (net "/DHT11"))
 (segment (start 166.700355 72.761813) (end 165.444565 72.761813) (width 0.2) (layer "F.Cu") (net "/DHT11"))
 (segment (start 142 71.537) (end 142 70.395786) (width 0.2) (layer "F.Cu") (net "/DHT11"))
 (segment (start 168.424355 71.037813) (end 166.700355 72.761813) (width 0.2) (layer "F.Cu") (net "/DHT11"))
 (segment (start 165.444565 72.761813) (end 163.720565 71.037813) (width 0.2) (layer "F.Cu") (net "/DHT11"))
 (segment (start 143.4 60.665686) (end 143.4 56.063654) (width 0.2) (layer "F.Cu") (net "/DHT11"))
 (segment (start 190.22246 78.72246) (end 190.22246 73.22246) (width 0.2) (layer "F.Cu") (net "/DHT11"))
 (segment (start 155.5 55) (end 156.8275 53.6725) (width 0.2) (layer "F.Cu") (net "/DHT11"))
 (segment (start 191.47246 79.319813) (end 190.819813 79.319813) (width 0.2) (layer "F.Cu") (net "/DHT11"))
 (segment (start 157.462187 71.037813) (end 155.284 73.216) (width 0.2) (layer "F.Cu") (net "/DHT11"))
 (segment (start 190.819813 79.319813) (end 190.22246 78.72246) (width 0.2) (layer "F.Cu") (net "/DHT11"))
 (segment (start 142 70.395786) (end 141 69.395786) (width 0.2) (layer "F.Cu") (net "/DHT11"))
 (segment (start 155.284 73.216) (end 155.284 74.227346) (width 0.2) (layer "F.Cu") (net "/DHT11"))
 (segment (start 156.8275 53.6725) (end 156.8275 51.4025) (width 0.2) (layer "F.Cu") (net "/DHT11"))
 (segment (start 141.5 62.69) (end 141.5 62.565686) (width 0.2) (layer "F.Cu") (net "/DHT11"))
 (segment (start 154.610346 74.901) (end 145.364 74.901) (width 0.2) (layer "F.Cu") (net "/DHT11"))
 (segment (start 188.037813 71.037813) (end 168.424355 71.037813) (width 0.2) (layer "F.Cu") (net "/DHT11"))
 (segment (start 155.284 74.227346) (end 154.610346 74.901) (width 0.2) (layer "F.Cu") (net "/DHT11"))
 (segment (start 189.82246 79.359708) (end 189.82246 73.388146) (width 0.2) (layer "F.Cu") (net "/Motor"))
 (segment (start 163.5 71.5) (end 157.565686 71.5) (width 0.2) (layer "F.Cu") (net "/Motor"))
 (segment (start 165.161813 73.161813) (end 163.5 71.5) (width 0.2) (layer "F.Cu") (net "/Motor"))
 (segment (start 180.403498 71.437813) (end 168.590041 71.437813) (width 0.2) (layer "F.Cu") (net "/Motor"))
 (segment (start 154.776031 75.301) (end 145.198314 75.301) (width 0.2) (layer "F.Cu") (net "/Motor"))
 (segment (start 155.684 73.381686) (end 155.684 74.393032) (width 0.2) (layer "F.Cu") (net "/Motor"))
 (segment (start 191.47246 81.009708) (end 189.82246 79.359708) (width 0.2) (layer "F.Cu") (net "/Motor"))
 (segment (start 166.86604 73.161813) (end 165.161813 73.161813) (width 0.2) (layer "F.Cu") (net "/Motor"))
 (segment (start 189.82246 73.388146) (end 187.934314 71.5) (width 0.2) (layer "F.Cu") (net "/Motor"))
 (segment (start 140.585786 71.81) (end 139.585786 70.81) (width 0.2) (layer "F.Cu") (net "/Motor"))
 (segment (start 157.565686 71.5) (end 155.684 73.381686) (width 0.2) (layer "F.Cu") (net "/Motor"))
 (segment (start 187.934314 71.5) (end 180.465685 71.5) (width 0.2) (layer "F.Cu") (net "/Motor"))
 (segment (start 155.684 74.393032) (end 154.776031 75.301) (width 0.2) (layer "F.Cu") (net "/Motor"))
 (segment (start 191.47246 81.859813) (end 191.47246 81.009708) (width 0.2) (layer "F.Cu") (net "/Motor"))
 (segment (start 139.585786 70.81) (end 138 70.81) (width 0.2) (layer "F.Cu") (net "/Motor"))
 (segment (start 180.465685 71.5) (end 180.403498 71.437813) (width 0.2) (layer "F.Cu") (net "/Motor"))
 (segment (start 141.707314 71.81) (end 140.585786 71.81) (width 0.2) (layer "F.Cu") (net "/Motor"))
 (segment (start 145.198314 75.301) (end 141.707314 71.81) (width 0.2) (layer "F.Cu") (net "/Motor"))
 (segment (start 168.590041 71.437813) (end 166.86604 73.161813) (width 0.2) (layer "F.Cu") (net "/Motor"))
 (segment (start 198.42 97.54) (end 195.38 94.5) (width 0.2) (layer "F.Cu") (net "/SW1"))
 (segment (start 195.38 94.5) (end 171.658333 94.5) (width 0.2) (layer "F.Cu") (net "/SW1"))
 (segment (start 171.658333 94.5) (end 167.32246 90.164127) (width 0.2) (layer "F.Cu") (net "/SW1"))
 (segment (start 167.32246 89.039918) (end 166.07246 87.789918) (width 0.2) (layer "F.Cu") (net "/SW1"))
 (segment (start 167.32246 90.164127) (end 167.32246 89.039918) (width 0.2) (layer "F.Cu") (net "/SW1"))
 (segment (start 166.07246 87.789918) (end 166.07246 86.939813) (width 0.2) (layer "F.Cu") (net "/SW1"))
 (segment (start 159.986587 95) (end 164.82246 90.164127) (width 0.2) (layer "F.Cu") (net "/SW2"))
 (segment (start 164.82246 83.959918) (end 166.07246 82.709918) (width 0.2) (layer "F.Cu") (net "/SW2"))
 (segment (start 164.82246 90.164127) (end 164.82246 83.959918) (width 0.2) (layer "F.Cu") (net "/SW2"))
 (segment (start 128.75 95) (end 159.986587 95) (width 0.2) (layer "F.Cu") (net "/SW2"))
 (segment (start 166.07246 82.709918) (end 166.07246 81.859813) (width 0.2) (layer "F.Cu") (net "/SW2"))
 (segment (start 140.420101 72.21) (end 141.541628 72.21) (width 0.2) (layer "F.Cu") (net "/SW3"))
 (segment (start 131.33 65.554214) (end 137.585786 71.81) (width 0.2) (layer "F.Cu") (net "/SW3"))
 (segment (start 138.724214 71.5) (end 139.710101 71.5) (width 0.2) (layer "F.Cu") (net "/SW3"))
 (segment (start 138.414214 71.81) (end 138.724214 71.5) (width 0.2) (layer "F.Cu") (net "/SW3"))
 (segment (start 148.651441 79.319813) (end 166.07246 79.319813) (width 0.2) (layer "F.Cu") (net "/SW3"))
 (segment (start 137.585786 71.81) (end 138.414214 71.81) (width 0.2) (layer "F.Cu") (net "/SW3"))
 (segment (start 139.710101 71.5) (end 140.420101 72.21) (width 0.2) (layer "F.Cu") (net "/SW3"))
 (segment (start 131.33 60.62) (end 131.33 65.554214) (width 0.2) (layer "F.Cu") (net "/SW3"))
 (segment (start 141.541628 72.21) (end 148.651441 79.319813) (width 0.2) (layer "F.Cu") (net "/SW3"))
 (segment (start 190.844565 80.797813) (end 190.22246 81.419918) (width 0.2) (layer "B.Cu") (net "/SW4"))
 (segment (start 168.021813 82.521813) (end 167.32246 81.82246) (width 0.2) (layer "B.Cu") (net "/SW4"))
 (segment (start 198.46 59.198168) (end 192.100355 65.557813) (width 0.2) (layer "B.Cu") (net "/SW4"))
 (segment (start 167.32246 78.029813) (end 166.07246 76.779813) (width 0.2) (layer "B.Cu") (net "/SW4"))
 (segment (start 192.100355 65.557813) (end 190.844565 65.557813) (width 0.2) (layer "B.Cu") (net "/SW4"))
 (segment (start 166.07246 76.779813) (end 168.220187 76.779813) (width 0.2) (layer "B.Cu") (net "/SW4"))
 (segment (start 191.684355 80.797813) (end 190.844565 80.797813) (width 0.2) (layer "B.Cu") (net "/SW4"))
 (segment (start 167.32246 81.82246) (end 167.32246 78.029813) (width 0.2) (layer "B.Cu") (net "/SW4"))
 (segment (start 198.46 55.4) (end 198.46 59.198168) (width 0.2) (layer "B.Cu") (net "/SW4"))
 (segment (start 190.22246 81.419918) (end 190.22246 81.77754) (width 0.2) (layer "B.Cu") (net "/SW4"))
 (segment (start 189 67.402378) (end 189 78.537248) (width 0.2) (layer "B.Cu") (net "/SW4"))
 (segment (start 189 78.537248) (end 190.844565 80.381813) (width 0.2) (layer "B.Cu") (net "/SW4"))
 (segment (start 190.22246 81.77754) (end 189.478187 82.521813) (width 0.2) (layer "B.Cu") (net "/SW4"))
 (segment (start 190.844565 80.381813) (end 191.268355 80.381813) (width 0.2) (layer "B.Cu") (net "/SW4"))
 (segment (start 191.268355 80.381813) (end 191.684355 80.797813) (width 0.2) (layer "B.Cu") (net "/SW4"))
 (segment (start 190.844565 65.557813) (end 189 67.402378) (width 0.2) (layer "B.Cu") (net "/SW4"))
 (segment (start 189.478187 82.521813) (end 168.021813 82.521813) (width 0.2) (layer "B.Cu") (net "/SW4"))
 (segment (start 161.5 49.510075) (end 163.52 51.530075) (width 0.2) (layer "B.Cu") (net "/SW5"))
 (segment (start 161.5 44.04) (end 161.5 49.510075) (width 0.2) (layer "B.Cu") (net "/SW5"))
 (segment (start 163.52 51.530075) (end 163.52 71.687353) (width 0.2) (layer "B.Cu") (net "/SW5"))
 (segment (start 162.46 43.08) (end 161.5 44.04) (width 0.2) (layer "B.Cu") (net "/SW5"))
 (segment (start 163.52 71.687353) (end 166.07246 74.239813) (width 0.2) (layer "B.Cu") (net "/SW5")))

